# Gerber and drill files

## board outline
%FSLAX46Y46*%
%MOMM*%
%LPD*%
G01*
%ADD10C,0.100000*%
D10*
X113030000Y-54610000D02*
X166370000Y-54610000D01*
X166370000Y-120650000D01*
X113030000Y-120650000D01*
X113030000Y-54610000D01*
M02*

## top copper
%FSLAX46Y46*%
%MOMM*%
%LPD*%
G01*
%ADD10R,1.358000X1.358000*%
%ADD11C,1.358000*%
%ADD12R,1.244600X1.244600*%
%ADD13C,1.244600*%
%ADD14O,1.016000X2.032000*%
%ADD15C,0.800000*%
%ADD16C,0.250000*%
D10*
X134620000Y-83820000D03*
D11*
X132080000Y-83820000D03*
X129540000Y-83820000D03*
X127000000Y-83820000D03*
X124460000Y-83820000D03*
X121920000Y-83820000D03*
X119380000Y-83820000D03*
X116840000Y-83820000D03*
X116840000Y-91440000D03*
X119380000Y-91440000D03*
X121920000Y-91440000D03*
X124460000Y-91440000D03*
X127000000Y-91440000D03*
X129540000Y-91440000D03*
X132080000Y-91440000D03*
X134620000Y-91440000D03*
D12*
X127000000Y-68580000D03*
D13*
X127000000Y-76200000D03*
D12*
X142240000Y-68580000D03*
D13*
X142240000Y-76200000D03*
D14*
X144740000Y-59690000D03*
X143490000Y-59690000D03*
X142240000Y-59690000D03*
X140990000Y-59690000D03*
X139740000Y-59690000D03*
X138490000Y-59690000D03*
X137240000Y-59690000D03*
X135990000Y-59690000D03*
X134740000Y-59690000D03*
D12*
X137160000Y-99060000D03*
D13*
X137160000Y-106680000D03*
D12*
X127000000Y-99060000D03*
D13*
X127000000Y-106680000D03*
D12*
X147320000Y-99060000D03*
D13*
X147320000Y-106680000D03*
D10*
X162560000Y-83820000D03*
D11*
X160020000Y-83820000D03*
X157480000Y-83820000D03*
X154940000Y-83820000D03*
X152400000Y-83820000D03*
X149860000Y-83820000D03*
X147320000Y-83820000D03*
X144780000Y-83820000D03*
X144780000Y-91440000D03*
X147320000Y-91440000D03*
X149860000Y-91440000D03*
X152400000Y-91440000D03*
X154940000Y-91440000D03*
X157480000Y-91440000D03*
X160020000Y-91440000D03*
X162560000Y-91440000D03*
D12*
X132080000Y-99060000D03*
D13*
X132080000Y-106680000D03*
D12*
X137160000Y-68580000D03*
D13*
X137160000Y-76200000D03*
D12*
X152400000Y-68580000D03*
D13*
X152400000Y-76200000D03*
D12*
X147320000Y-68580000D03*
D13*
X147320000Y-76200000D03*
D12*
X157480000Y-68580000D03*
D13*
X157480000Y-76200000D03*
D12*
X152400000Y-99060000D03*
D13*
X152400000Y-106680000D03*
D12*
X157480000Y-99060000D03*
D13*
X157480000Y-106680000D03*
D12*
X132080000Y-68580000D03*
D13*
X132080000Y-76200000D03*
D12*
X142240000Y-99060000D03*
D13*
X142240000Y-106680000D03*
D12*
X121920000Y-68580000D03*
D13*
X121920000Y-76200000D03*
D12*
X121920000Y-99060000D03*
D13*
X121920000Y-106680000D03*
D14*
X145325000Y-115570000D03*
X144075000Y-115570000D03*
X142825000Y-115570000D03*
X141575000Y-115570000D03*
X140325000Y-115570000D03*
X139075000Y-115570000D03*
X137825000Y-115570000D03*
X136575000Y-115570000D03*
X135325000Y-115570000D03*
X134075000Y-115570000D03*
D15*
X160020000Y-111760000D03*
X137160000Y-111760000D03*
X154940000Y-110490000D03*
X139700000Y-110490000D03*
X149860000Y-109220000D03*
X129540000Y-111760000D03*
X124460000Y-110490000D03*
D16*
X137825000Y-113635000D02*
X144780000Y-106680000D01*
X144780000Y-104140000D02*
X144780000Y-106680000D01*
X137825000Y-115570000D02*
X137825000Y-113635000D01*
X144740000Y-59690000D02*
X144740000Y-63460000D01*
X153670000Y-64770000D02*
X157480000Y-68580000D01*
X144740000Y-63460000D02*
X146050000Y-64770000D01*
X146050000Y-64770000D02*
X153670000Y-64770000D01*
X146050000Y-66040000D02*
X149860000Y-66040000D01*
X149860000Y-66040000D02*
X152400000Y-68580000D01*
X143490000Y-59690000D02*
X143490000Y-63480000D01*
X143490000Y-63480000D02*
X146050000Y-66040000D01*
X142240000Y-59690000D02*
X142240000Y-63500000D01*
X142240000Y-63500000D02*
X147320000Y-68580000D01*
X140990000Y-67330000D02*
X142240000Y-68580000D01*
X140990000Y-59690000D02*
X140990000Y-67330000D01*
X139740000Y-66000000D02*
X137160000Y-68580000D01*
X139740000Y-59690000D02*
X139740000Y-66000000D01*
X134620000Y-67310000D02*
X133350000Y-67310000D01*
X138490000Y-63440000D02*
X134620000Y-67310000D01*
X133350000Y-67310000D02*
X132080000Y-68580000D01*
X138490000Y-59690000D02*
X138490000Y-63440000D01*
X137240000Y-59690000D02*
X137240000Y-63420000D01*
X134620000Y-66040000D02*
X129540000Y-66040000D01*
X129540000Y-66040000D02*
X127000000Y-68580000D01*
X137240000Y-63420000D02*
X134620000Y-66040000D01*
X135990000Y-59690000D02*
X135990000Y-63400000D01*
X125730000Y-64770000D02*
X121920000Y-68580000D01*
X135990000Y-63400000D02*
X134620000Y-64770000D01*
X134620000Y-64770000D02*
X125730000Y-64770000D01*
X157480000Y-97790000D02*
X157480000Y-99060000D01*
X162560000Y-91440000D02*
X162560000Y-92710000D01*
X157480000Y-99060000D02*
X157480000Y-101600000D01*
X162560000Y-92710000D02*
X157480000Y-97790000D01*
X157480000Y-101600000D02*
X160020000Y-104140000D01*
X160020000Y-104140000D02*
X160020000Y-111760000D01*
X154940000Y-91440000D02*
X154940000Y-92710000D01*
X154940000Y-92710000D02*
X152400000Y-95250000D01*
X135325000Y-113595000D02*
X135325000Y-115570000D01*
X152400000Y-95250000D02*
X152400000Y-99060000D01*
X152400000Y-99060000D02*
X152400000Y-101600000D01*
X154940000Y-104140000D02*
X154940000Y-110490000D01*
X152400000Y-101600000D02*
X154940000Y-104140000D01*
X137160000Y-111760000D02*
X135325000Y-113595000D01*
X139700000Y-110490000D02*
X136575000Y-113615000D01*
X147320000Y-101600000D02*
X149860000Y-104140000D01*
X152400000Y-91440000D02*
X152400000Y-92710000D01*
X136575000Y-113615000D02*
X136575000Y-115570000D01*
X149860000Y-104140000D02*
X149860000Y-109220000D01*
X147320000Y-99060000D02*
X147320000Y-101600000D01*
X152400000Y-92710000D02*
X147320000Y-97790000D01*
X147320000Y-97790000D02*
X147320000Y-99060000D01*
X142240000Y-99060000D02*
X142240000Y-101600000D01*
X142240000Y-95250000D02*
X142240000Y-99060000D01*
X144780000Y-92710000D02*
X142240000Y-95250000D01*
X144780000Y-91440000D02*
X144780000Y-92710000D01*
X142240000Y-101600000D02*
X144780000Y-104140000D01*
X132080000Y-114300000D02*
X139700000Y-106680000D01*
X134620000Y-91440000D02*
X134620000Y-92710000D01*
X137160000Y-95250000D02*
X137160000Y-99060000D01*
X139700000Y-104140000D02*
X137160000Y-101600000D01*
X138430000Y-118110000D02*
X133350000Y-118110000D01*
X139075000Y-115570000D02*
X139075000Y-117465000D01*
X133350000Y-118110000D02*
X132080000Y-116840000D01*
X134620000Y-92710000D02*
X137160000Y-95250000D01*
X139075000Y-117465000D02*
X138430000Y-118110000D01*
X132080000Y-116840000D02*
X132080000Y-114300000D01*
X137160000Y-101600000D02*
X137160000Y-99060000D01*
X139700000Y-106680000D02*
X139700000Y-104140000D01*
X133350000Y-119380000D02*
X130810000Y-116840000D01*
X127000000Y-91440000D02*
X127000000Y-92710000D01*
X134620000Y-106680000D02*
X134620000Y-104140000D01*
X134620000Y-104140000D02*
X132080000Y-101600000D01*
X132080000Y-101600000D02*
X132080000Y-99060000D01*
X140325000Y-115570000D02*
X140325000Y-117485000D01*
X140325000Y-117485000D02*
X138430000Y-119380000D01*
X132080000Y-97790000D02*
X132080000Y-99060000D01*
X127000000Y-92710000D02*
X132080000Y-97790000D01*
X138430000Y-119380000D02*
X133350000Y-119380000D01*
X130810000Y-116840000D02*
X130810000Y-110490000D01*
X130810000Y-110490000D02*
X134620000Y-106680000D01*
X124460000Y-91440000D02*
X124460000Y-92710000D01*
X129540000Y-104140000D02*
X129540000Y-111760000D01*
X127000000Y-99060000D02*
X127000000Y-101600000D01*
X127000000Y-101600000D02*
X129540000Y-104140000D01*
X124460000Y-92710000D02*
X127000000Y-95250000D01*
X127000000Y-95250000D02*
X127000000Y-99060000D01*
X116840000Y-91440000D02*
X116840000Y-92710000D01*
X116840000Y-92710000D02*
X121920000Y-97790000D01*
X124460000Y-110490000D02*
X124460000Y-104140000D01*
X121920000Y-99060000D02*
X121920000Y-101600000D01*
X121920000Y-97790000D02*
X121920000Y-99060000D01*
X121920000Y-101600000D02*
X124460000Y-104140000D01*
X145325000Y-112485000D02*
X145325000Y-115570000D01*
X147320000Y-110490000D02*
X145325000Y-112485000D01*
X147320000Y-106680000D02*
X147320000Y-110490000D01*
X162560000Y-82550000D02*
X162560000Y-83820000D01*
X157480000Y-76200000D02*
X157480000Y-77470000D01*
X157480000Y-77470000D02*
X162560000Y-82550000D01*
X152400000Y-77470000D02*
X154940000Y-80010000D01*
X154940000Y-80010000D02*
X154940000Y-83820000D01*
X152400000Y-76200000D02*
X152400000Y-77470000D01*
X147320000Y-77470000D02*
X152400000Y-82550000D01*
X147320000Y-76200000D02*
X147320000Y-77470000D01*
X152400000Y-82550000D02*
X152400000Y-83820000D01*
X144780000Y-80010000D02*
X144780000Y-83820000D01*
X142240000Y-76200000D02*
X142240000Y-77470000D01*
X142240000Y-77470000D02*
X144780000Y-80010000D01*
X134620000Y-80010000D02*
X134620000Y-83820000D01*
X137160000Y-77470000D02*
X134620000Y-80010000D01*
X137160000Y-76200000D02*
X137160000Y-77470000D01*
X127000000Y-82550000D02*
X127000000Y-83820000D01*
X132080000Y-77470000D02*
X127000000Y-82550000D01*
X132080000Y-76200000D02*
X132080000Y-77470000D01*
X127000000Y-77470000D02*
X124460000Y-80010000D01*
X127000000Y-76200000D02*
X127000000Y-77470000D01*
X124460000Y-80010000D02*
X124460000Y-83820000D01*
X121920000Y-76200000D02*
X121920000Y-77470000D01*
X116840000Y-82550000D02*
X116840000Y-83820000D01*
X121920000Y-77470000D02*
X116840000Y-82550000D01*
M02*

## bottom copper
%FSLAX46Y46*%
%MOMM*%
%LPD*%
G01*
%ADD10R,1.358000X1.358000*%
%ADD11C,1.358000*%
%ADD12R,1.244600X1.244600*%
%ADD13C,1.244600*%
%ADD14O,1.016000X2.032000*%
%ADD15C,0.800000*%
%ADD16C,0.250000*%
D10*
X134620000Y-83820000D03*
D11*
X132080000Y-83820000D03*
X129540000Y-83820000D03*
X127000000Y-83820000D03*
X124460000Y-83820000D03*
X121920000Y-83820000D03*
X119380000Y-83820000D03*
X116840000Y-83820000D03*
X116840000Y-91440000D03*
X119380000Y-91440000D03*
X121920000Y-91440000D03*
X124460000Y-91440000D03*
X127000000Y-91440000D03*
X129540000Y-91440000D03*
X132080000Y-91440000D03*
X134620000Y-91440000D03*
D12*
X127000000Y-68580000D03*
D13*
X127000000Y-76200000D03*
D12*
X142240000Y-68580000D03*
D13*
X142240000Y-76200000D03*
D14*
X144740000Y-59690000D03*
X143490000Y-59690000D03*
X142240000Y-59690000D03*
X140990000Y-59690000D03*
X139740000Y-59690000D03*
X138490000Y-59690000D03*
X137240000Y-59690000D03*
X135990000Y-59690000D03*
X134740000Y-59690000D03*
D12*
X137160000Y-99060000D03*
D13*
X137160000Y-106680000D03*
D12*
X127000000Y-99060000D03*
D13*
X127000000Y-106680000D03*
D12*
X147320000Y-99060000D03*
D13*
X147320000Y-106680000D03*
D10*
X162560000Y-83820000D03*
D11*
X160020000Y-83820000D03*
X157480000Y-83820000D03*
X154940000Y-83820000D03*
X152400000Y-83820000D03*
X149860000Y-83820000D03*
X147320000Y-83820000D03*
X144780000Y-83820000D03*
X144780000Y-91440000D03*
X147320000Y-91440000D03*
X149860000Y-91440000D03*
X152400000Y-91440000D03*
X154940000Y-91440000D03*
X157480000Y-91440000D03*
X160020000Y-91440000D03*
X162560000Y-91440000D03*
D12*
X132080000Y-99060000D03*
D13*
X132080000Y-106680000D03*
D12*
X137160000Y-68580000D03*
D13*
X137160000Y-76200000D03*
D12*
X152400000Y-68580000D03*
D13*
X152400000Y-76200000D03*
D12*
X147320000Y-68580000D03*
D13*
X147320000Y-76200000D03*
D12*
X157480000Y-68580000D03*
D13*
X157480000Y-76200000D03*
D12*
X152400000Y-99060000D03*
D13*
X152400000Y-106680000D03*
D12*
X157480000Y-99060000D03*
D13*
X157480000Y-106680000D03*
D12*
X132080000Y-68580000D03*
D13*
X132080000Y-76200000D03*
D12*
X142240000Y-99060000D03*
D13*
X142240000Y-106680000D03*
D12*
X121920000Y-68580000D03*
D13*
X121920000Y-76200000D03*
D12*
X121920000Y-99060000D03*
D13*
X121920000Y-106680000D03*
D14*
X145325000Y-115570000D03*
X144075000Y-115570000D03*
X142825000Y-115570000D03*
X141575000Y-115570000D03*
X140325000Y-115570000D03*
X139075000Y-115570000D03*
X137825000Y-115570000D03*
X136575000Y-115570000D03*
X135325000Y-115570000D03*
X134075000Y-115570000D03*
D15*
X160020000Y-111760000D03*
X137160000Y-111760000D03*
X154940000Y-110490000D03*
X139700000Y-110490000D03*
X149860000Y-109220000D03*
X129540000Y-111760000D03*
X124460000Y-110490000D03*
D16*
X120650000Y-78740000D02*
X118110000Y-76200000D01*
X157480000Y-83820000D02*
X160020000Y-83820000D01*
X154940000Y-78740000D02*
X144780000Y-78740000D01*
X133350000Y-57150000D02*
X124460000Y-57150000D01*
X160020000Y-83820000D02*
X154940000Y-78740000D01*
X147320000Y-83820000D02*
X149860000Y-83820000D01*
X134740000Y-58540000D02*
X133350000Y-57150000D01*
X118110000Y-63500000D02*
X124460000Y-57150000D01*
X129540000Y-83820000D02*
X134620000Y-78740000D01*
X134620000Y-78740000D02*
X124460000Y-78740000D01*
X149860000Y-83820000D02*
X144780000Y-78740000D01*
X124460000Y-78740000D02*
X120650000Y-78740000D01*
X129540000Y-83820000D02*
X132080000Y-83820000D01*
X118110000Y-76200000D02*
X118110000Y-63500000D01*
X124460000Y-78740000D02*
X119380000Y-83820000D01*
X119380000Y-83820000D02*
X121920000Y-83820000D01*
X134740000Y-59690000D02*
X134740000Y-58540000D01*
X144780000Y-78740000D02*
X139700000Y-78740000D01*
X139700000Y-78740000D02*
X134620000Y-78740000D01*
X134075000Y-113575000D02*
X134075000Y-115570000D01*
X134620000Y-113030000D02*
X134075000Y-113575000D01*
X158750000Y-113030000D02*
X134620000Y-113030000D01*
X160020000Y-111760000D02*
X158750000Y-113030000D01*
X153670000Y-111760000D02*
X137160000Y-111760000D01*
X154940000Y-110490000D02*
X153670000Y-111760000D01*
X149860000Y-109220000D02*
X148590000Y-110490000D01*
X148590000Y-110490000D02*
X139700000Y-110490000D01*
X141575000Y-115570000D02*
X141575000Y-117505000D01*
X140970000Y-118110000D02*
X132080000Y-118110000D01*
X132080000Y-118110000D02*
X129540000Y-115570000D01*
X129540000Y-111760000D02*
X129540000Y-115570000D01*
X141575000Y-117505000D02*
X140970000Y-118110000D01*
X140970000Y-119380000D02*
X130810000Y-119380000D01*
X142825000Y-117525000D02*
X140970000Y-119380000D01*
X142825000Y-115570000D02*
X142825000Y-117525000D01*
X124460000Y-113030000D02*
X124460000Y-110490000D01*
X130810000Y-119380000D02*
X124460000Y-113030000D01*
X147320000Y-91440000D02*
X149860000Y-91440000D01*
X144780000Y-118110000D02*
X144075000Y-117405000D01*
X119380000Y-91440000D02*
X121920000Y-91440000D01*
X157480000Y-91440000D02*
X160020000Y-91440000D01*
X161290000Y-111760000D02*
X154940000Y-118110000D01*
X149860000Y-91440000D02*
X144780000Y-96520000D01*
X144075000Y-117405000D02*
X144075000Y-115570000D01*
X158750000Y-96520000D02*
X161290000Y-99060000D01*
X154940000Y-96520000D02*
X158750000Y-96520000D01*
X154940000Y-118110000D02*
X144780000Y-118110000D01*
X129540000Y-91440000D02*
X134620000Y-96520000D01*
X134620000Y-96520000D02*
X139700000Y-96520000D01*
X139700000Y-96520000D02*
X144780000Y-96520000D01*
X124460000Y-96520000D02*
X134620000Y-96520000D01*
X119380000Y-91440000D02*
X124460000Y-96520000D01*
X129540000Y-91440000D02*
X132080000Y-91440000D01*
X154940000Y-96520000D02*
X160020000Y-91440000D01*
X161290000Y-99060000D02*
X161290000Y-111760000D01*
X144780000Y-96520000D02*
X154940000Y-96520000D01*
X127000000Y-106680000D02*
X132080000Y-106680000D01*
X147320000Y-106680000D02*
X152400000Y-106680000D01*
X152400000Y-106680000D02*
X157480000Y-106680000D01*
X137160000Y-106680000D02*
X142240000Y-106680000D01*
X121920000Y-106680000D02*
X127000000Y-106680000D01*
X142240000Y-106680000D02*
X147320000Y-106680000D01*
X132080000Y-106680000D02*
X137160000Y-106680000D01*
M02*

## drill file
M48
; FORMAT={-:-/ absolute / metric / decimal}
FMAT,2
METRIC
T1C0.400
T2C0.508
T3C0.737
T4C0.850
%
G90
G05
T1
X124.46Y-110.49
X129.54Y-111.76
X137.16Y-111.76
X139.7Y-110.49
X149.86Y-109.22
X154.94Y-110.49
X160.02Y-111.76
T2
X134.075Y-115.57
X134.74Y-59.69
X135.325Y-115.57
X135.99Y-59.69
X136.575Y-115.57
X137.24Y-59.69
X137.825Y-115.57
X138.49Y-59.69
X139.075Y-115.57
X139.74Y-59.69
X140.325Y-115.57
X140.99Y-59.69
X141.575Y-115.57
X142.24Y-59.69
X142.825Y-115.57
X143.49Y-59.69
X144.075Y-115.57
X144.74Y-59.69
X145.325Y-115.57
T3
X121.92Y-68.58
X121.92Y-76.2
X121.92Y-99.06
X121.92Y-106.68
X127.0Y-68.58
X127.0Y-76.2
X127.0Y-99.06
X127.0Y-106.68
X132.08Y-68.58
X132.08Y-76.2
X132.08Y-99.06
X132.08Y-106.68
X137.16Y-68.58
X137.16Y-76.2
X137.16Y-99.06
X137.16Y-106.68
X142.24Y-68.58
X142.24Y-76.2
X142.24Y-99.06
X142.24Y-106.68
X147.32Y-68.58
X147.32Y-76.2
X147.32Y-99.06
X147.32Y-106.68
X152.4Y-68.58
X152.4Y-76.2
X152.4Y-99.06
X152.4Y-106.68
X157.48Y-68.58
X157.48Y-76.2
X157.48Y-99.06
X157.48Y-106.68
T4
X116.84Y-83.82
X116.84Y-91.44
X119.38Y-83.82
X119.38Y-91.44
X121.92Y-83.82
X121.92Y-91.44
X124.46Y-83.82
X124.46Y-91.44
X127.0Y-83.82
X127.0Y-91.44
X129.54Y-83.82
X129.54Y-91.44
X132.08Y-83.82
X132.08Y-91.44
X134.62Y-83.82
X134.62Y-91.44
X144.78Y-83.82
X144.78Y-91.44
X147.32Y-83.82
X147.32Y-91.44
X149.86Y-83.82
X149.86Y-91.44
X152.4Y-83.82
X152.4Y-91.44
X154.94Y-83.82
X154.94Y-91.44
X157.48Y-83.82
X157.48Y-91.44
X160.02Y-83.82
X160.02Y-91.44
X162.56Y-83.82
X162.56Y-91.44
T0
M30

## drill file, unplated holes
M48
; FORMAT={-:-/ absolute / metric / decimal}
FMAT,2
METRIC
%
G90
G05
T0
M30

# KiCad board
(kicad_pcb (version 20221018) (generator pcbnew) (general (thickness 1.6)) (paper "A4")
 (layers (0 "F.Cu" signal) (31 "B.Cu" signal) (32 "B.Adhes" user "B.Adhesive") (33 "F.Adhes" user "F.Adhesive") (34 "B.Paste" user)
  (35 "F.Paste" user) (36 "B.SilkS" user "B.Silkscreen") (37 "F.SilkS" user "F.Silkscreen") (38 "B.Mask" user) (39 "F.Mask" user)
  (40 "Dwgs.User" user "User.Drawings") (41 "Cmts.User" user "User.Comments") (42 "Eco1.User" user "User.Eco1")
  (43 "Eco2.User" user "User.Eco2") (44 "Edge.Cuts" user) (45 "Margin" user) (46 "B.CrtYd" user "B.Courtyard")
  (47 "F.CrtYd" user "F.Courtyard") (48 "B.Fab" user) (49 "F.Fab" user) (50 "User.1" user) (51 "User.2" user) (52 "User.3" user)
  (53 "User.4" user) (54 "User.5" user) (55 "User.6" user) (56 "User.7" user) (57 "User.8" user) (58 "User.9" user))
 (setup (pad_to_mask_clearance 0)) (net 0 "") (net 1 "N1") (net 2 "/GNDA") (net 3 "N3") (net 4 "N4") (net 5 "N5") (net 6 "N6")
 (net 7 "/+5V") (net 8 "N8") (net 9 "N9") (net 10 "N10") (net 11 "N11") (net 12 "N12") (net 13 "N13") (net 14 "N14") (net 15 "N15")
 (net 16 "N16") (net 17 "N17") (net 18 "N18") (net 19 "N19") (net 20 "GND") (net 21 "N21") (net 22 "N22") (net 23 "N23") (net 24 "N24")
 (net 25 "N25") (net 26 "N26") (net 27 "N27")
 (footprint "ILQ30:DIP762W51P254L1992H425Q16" (layer "F.Cu") (at 125.73 87.63 -90)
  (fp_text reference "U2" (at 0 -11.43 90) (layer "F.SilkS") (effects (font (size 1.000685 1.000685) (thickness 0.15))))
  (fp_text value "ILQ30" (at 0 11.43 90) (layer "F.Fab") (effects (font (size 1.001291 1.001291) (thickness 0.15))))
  (pad "1" thru_hole rect (at -3.81 -8.89 270) (size 1.358 1.358) (drill 0.85) (layers "*.Cu" "*.Mask") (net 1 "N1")
   (solder_mask_margin 0.102))
  (pad "2" thru_hole circle (at -3.81 -6.35 270) (size 1.358 1.358) (drill 0.85) (layers "*.Cu" "*.Mask") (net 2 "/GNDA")
   (solder_mask_margin 0.102))
  (pad "3" thru_hole circle (at -3.81 -3.81 270) (size 1.358 1.358) (drill 0.85) (layers "*.Cu" "*.Mask") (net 2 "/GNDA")
   (solder_mask_margin 0.102))
  (pad "4" thru_hole circle (at -3.81 -1.27 270) (size 1.358 1.358) (drill 0.85) (layers "*.Cu" "*.Mask") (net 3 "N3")
   (solder_mask_margin 0.102))
  (pad "5" thru_hole circle (at -3.81 1.27 270) (size 1.358 1.358) (drill 0.85) (layers "*.Cu" "*.Mask") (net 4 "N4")
   (solder_mask_margin 0.102))
  (pad "6" thru_hole circle (at -3.81 3.81 270) (size 1.358 1.358) (drill 0.85) (layers "*.Cu" "*.Mask") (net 2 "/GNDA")
   (solder_mask_margin 0.102))
  (pad "7" thru_hole circle (at -3.81 6.35 270) (size 1.358 1.358) (drill 0.85) (layers "*.Cu" "*.Mask") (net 2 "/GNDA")
   (solder_mask_margin 0.102))
  (pad "8" thru_hole circle (at -3.81 8.89 270) (size 1.358 1.358) (drill 0.85) (layers "*.Cu" "*.Mask") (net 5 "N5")
   (solder_mask_margin 0.102))
  (pad "9" thru_hole circle (at 3.81 8.89 270) (size 1.358 1.358) (drill 0.85) (layers "*.Cu" "*.Mask") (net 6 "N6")
   (solder_mask_margin 0.102))
  (pad "10" thru_hole circle (at 3.81 6.35 270) (size 1.358 1.358) (drill 0.85) (layers "*.Cu" "*.Mask") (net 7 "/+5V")
   (solder_mask_margin 0.102))
  (pad "11" thru_hole circle (at 3.81 3.81 270) (size 1.358 1.358) (drill 0.85) (layers "*.Cu" "*.Mask") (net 7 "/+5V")
   (solder_mask_margin 0.102))
  (pad "12" thru_hole circle (at 3.81 1.27 270) (size 1.358 1.358) (drill 0.85) (layers "*.Cu" "*.Mask") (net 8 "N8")
   (solder_mask_margin 0.102))
  (pad "13" thru_hole circle (at 3.81 -1.27 270) (size 1.358 1.358) (drill 0.85) (layers "*.Cu" "*.Mask") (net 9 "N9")
   (solder_mask_margin 0.102))
  (pad "14" thru_hole circle (at 3.81 -3.81 270) (size 1.358 1.358) (drill 0.85) (layers "*.Cu" "*.Mask") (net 7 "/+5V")
   (solder_mask_margin 0.102))
  (pad "15" thru_hole circle (at 3.81 -6.35 270) (size 1.358 1.358) (drill 0.85) (layers "*.Cu" "*.Mask") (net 7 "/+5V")
   (solder_mask_margin 0.102))
  (pad "16" thru_hole circle (at 3.81 -8.89 270) (size 1.358 1.358) (drill 0.85) (layers "*.Cu" "*.Mask") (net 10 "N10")
   (solder_mask_margin 0.102)))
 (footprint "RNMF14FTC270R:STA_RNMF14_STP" (layer "F.Cu") (at 127 68.58 -90)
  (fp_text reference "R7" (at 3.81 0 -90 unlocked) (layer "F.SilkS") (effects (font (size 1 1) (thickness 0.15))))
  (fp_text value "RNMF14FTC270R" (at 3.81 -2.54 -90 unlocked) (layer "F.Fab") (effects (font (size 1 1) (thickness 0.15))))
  (pad "1" thru_hole rect (at 0 0 270) (size 1.2446 1.2446) (drill 0.7366) (layers "*.Cu" "*.Mask") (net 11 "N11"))
  (pad "2" thru_hole circle (at 7.62 0 270) (size 1.2446 1.2446) (drill 0.7366) (layers "*.Cu" "*.Mask") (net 4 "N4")))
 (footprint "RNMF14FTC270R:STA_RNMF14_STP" (layer "F.Cu") (at 142.24 68.58 -90)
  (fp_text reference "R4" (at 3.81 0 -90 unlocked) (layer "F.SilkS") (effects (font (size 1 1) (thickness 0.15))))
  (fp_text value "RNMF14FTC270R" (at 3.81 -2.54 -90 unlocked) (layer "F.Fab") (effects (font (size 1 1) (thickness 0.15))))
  (pad "1" thru_hole rect (at 0 0 270) (size 1.2446 1.2446) (drill 0.7366) (layers "*.Cu" "*.Mask") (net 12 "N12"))
  (pad "2" thru_hole circle (at 7.62 0 270) (size 1.2446 1.2446) (drill 0.7366) (layers "*.Cu" "*.Mask") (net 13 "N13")))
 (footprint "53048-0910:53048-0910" (layer "F.Cu") (at 139.74 59.69 180)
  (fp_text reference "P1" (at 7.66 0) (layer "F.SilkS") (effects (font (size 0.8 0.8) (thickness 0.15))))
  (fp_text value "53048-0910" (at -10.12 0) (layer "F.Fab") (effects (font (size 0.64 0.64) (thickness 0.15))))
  (pad "1" thru_hole oval (at -5 0 180) (size 1.016 2.032) (drill 0.508) (layers "*.Cu" "*.Mask") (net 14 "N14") (solder_mask_margin 0.102))
  (pad "2" thru_hole oval (at -3.75 0 180) (size 1.016 2.032) (drill 0.508) (layers "*.Cu" "*.Mask") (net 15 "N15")
   (solder_mask_margin 0.102))
  (pad "3" thru_hole oval (at -2.5 0 180) (size 1.016 2.032) (drill 0.508) (layers "*.Cu" "*.Mask") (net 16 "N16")
   (solder_mask_margin 0.102))
  (pad "4" thru_hole oval (at -1.25 0 180) (size 1.016 2.032) (drill 0.508) (layers "*.Cu" "*.Mask") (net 12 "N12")
   (solder_mask_margin 0.102))
  (pad "5" thru_hole oval (at 0 0 180) (size 1.016 2.032) (drill 0.508) (layers "*.Cu" "*.Mask") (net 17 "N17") (solder_mask_margin 0.102))
  (pad "6" thru_hole oval (at 1.25 0 180) (size 1.016 2.032) (drill 0.508) (layers "*.Cu" "*.Mask") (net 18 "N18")
   (solder_mask_margin 0.102))
  (pad "7" thru_hole oval (at 2.5 0 180) (size 1.016 2.032) (drill 0.508) (layers "*.Cu" "*.Mask") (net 11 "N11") (solder_mask_margin 0.102))
  (pad "8" thru_hole oval (at 3.75 0 180) (size 1.016 2.032) (drill 0.508) (layers "*.Cu" "*.Mask") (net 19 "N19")
   (solder_mask_margin 0.102))
  (pad "9" thru_hole oval (at 5 0 180) (size 1.016 2.032) (drill 0.508) (layers "*.Cu" "*.Mask") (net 2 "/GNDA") (solder_mask_margin 0.102)))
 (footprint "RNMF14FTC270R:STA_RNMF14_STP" (layer "F.Cu") (at 137.16 99.06 -90)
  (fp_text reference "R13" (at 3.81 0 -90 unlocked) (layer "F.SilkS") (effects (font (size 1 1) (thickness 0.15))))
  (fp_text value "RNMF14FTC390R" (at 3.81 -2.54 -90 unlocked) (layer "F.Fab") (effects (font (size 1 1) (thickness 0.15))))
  (pad "1" thru_hole rect (at 0 0 270) (size 1.2446 1.2446) (drill 0.7366) (layers "*.Cu" "*.Mask") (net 10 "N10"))
  (pad "2" thru_hole circle (at 7.62 0 270) (size 1.2446 1.2446) (drill 0.7366) (layers "*.Cu" "*.Mask") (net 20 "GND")))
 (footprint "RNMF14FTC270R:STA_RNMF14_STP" (layer "F.Cu") (at 127 99.06 -90)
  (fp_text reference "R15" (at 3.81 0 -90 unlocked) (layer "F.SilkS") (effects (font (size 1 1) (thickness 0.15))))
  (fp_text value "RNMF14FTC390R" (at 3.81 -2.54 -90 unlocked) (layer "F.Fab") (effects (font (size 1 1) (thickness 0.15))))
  (pad "1" thru_hole rect (at 0 0 270) (size 1.2446 1.2446) (drill 0.7366) (layers "*.Cu" "*.Mask") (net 8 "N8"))
  (pad "2" thru_hole circle (at 7.62 0 270) (size 1.2446 1.2446) (drill 0.7366) (layers "*.Cu" "*.Mask") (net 20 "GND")))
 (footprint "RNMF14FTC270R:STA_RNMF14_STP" (layer "F.Cu") (at 147.32 99.06 -90)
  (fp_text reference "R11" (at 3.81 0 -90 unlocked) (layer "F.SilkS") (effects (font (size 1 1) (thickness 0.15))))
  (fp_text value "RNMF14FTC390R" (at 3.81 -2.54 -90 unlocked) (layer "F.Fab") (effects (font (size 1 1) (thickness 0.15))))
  (pad "1" thru_hole rect (at 0 0 270) (size 1.2446 1.2446) (drill 0.7366) (layers "*.Cu" "*.Mask") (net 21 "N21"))
  (pad "2" thru_hole circle (at 7.62 0 270) (size 1.2446 1.2446) (drill 0.7366) (layers "*.Cu" "*.Mask") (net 20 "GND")))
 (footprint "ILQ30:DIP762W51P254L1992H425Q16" (layer "F.Cu") (at 153.67 87.63 -90)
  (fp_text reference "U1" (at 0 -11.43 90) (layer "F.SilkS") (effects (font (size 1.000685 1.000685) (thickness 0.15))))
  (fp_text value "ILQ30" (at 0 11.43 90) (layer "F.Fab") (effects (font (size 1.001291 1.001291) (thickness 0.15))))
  (pad "1" thru_hole rect (at -3.81 -8.89 270) (size 1.358 1.358) (drill 0.85) (layers "*.Cu" "*.Mask") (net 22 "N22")
   (solder_mask_margin 0.102))
  (pad "2" thru_hole circle (at -3.81 -6.35 270) (size 1.358 1.358) (drill 0.85) (layers "*.Cu" "*.Mask") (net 2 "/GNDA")
   (solder_mask_margin 0.102))
  (pad "3" thru_hole circle (at -3.81 -3.81 270) (size 1.358 1.358) (drill 0.85) (layers "*.Cu" "*.Mask") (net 2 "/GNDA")
   (solder_mask_margin 0.102))
  (pad "4" thru_hole circle (at -3.81 -1.27 270) (size 1.358 1.358) (drill 0.85) (layers "*.Cu" "*.Mask") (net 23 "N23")
   (solder_mask_margin 0.102))
  (pad "5" thru_hole circle (at -3.81 1.27 270) (size 1.358 1.358) (drill 0.85) (layers "*.Cu" "*.Mask") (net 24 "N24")
   (solder_mask_margin 0.102))
  (pad "6" thru_hole circle (at -3.81 3.81 270) (size 1.358 1.358) (drill 0.85) (layers "*.Cu" "*.Mask") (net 2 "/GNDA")
   (solder_mask_margin 0.102))
  (pad "7" thru_hole circle (at -3.81 6.35 270) (size 1.358 1.358) (drill 0.85) (layers "*.Cu" "*.Mask") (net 2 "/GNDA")
   (solder_mask_margin 0.102))
  (pad "8" thru_hole circle (at -3.81 8.89 270) (size 1.358 1.358) (drill 0.85) (layers "*.Cu" "*.Mask") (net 13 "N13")
   (solder_mask_margin 0.102))
  (pad "9" thru_hole circle (at 3.81 8.89 270) (size 1.358 1.358) (drill 0.85) (layers "*.Cu" "*.Mask") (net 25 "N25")
   (solder_mask_margin 0.102))
  (pad "10" thru_hole circle (at 3.81 6.35 270) (size 1.358 1.358) (drill 0.85) (layers "*.Cu" "*.Mask") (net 7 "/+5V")
   (solder_mask_margin 0.102))
  (pad "11" thru_hole circle (at 3.81 3.81 270) (size 1.358 1.358) (drill 0.85) (layers "*.Cu" "*.Mask") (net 7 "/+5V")
   (solder_mask_margin 0.102))
  (pad "12" thru_hole circle (at 3.81 1.27 270) (size 1.358 1.358) (drill 0.85) (layers "*.Cu" "*.Mask") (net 21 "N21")
   (solder_mask_margin 0.102))
  (pad "13" thru_hole circle (at 3.81 -1.27 270) (size 1.358 1.358) (drill 0.85) (layers "*.Cu" "*.Mask") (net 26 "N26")
   (solder_mask_margin 0.102))
  (pad "14" thru_hole circle (at 3.81 -3.81 270) (size 1.358 1.358) (drill 0.85) (layers "*.Cu" "*.Mask") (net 7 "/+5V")
   (solder_mask_margin 0.102))
  (pad "15" thru_hole circle (at 3.81 -6.35 270) (size 1.358 1.358) (drill 0.85) (layers "*.Cu" "*.Mask") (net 7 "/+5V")
   (solder_mask_margin 0.102))
  (pad "16" thru_hole circle (at 3.81 -8.89 270) (size 1.358 1.358) (drill 0.85) (layers "*.Cu" "*.Mask") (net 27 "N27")
   (solder_mask_margin 0.102)))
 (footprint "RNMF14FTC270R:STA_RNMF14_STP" (layer "F.Cu") (at 132.08 99.06 -90)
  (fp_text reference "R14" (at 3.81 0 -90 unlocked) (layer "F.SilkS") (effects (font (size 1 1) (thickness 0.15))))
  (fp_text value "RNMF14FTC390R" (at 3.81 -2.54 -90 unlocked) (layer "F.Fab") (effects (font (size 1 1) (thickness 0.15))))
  (pad "1" thru_hole rect (at 0 0 270) (size 1.2446 1.2446) (drill 0.7366) (layers "*.Cu" "*.Mask") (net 9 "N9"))
  (pad "2" thru_hole circle (at 7.62 0 270) (size 1.2446 1.2446) (drill 0.7366) (layers "*.Cu" "*.Mask") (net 20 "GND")))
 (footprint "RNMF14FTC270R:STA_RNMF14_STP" (layer "F.Cu") (at 137.16 68.58 -90)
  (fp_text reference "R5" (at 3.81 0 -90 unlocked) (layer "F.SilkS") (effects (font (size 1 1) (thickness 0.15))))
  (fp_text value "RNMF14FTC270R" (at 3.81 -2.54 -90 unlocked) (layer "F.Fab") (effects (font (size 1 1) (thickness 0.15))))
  (pad "1" thru_hole rect (at 0 0 270) (size 1.2446 1.2446) (drill 0.7366) (layers "*.Cu" "*.Mask") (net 17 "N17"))
  (pad "2" thru_hole circle (at 7.62 0 270) (size 1.2446 1.2446) (drill 0.7366) (layers "*.Cu" "*.Mask") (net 1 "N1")))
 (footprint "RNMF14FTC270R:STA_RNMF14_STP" (layer "F.Cu") (at 152.4 68.58 -90)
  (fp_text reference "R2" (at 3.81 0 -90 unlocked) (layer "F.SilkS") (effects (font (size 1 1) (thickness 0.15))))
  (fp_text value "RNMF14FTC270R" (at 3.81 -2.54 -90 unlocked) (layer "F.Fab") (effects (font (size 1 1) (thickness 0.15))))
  (pad "1" thru_hole rect (at 0 0 270) (size 1.2446 1.2446) (drill 0.7366) (layers "*.Cu" "*.Mask") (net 15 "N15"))
  (pad "2" thru_hole circle (at 7.62 0 270) (size 1.2446 1.2446) (drill 0.7366) (layers "*.Cu" "*.Mask") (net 23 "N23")))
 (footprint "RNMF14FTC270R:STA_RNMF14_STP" (layer "F.Cu") (at 147.32 68.58 -90)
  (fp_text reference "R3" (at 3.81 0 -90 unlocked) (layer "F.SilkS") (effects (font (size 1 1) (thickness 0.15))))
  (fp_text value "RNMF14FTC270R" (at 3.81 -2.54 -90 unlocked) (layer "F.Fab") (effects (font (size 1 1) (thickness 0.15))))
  (pad "1" thru_hole rect (at 0 0 270) (size 1.2446 1.2446) (drill 0.7366) (layers "*.Cu" "*.Mask") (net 16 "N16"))
  (pad "2" thru_hole circle (at 7.62 0 270) (size 1.2446 1.2446) (drill 0.7366) (layers "*.Cu" "*.Mask") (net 24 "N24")))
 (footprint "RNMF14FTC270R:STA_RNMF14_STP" (layer "F.Cu") (at 157.48 68.58 -90)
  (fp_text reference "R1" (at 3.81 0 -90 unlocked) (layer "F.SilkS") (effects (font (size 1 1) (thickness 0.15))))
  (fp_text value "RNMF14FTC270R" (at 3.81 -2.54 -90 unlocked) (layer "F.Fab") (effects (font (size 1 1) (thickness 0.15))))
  (pad "1" thru_hole rect (at 0 0 270) (size 1.2446 1.2446) (drill 0.7366) (layers "*.Cu" "*.Mask") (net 14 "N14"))
  (pad "2" thru_hole circle (at 7.62 0 270) (size 1.2446 1.2446) (drill 0.7366) (layers "*.Cu" "*.Mask") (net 22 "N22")))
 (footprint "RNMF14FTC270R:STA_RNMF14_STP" (layer "F.Cu") (at 152.4 99.06 -90)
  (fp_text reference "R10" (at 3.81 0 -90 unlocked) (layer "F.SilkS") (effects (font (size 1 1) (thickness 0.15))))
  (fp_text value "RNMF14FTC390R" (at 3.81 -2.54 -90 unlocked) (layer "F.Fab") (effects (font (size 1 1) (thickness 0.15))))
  (pad "1" thru_hole rect (at 0 0 270) (size 1.2446 1.2446) (drill 0.7366) (layers "*.Cu" "*.Mask") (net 26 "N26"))
  (pad "2" thru_hole circle (at 7.62 0 270) (size 1.2446 1.2446) (drill 0.7366) (layers "*.Cu" "*.Mask") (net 20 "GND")))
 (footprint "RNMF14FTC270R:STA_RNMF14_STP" (layer "F.Cu") (at 157.48 99.06 -90)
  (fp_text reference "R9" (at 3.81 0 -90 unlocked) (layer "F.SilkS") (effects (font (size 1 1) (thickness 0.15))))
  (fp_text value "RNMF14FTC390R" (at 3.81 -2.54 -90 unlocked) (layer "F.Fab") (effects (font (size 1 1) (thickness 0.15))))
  (pad "1" thru_hole rect (at 0 0 270) (size 1.2446 1.2446) (drill 0.7366) (layers "*.Cu" "*.Mask") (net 27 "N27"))
  (pad "2" thru_hole circle (at 7.62 0 270) (size 1.2446 1.2446) (drill 0.7366) (layers "*.Cu" "*.Mask") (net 20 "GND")))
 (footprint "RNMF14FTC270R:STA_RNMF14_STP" (layer "F.Cu") (at 132.08 68.58 -90)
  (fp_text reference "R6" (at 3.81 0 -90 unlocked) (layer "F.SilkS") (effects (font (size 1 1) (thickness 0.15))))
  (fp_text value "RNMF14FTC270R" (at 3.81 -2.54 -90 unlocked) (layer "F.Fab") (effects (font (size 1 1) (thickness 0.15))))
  (pad "1" thru_hole rect (at 0 0 270) (size 1.2446 1.2446) (drill 0.7366) (layers "*.Cu" "*.Mask") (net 18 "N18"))
  (pad "2" thru_hole circle (at 7.62 0 270) (size 1.2446 1.2446) (drill 0.7366) (layers "*.Cu" "*.Mask") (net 3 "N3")))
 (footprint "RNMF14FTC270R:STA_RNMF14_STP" (layer "F.Cu") (at 142.24 99.06 -90)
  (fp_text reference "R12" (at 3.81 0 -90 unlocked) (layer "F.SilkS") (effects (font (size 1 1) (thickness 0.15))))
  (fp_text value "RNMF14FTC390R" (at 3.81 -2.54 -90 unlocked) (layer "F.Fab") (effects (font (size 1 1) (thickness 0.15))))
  (pad "1" thru_hole rect (at 0 0 270) (size 1.2446 1.2446) (drill 0.7366) (layers "*.Cu" "*.Mask") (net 25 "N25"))
  (pad "2" thru_hole circle (at 7.62 0 270) (size 1.2446 1.2446) (drill 0.7366) (layers "*.Cu" "*.Mask") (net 20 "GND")))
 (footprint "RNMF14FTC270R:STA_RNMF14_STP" (layer "F.Cu") (at 121.92 68.58 -90)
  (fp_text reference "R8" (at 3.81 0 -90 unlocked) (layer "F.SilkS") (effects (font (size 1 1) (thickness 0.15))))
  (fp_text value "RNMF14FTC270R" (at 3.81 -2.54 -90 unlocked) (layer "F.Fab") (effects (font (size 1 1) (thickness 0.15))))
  (pad "1" thru_hole rect (at 0 0 270) (size 1.2446 1.2446) (drill 0.7366) (layers "*.Cu" "*.Mask") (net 19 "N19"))
  (pad "2" thru_hole circle (at 7.62 0 270) (size 1.2446 1.2446) (drill 0.7366) (layers "*.Cu" "*.Mask") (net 5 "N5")))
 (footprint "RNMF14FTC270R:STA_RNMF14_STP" (layer "F.Cu") (at 121.92 99.06 -90)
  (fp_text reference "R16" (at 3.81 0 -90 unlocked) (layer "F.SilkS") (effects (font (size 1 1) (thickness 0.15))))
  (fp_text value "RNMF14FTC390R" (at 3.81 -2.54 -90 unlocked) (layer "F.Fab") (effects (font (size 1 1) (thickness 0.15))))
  (pad "1" thru_hole rect (at 0 0 270) (size 1.2446 1.2446) (drill 0.7366) (layers "*.Cu" "*.Mask") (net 6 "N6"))
  (pad "2" thru_hole circle (at 7.62 0 270) (size 1.2446 1.2446) (drill 0.7366) (layers "*.Cu" "*.Mask") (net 20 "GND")))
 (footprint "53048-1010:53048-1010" (layer "F.Cu") (at 139.7 115.57)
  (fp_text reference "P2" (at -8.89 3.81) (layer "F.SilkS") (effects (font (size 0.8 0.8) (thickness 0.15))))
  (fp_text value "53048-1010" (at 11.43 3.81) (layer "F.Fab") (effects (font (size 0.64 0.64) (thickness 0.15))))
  (pad "1" thru_hole oval (at -5.625 0) (size 1.016 2.032) (drill 0.508) (layers "*.Cu" "*.Mask") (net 27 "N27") (solder_mask_margin 0.102))
  (pad "2" thru_hole oval (at -4.375 0) (size 1.016 2.032) (drill 0.508) (layers "*.Cu" "*.Mask") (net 26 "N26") (solder_mask_margin 0.102))
  (pad "3" thru_hole oval (at -3.125 0) (size 1.016 2.032) (drill 0.508) (layers "*.Cu" "*.Mask") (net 21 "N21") (solder_mask_margin 0.102))
  (pad "4" thru_hole oval (at -1.875 0) (size 1.016 2.032) (drill 0.508) (layers "*.Cu" "*.Mask") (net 25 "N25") (solder_mask_margin 0.102))
  (pad "5" thru_hole oval (at -0.625 0) (size 1.016 2.032) (drill 0.508) (layers "*.Cu" "*.Mask") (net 10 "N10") (solder_mask_margin 0.102))
  (pad "6" thru_hole oval (at 0.625 0) (size 1.016 2.032) (drill 0.508) (layers "*.Cu" "*.Mask") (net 9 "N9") (solder_mask_margin 0.102))
  (pad "7" thru_hole oval (at 1.875 0) (size 1.016 2.032) (drill 0.508) (layers "*.Cu" "*.Mask") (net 8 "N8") (solder_mask_margin 0.102))
  (pad "8" thru_hole oval (at 3.125 0) (size 1.016 2.032) (drill 0.508) (layers "*.Cu" "*.Mask") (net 6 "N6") (solder_mask_margin 0.102))
  (pad "9" thru_hole oval (at 4.375 0) (size 1.016 2.032) (drill 0.508) (layers "*.Cu" "*.Mask") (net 7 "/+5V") (solder_mask_margin 0.102))
  (pad "10" thru_hole oval (at 5.625 0) (size 1.016 2.032) (drill 0.508) (layers "*.Cu" "*.Mask") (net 20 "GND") (solder_mask_margin 0.102)))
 (gr_rect (start 113.03 54.61) (end 166.37 120.65) (stroke (width 0.1) (type default)) (fill none) (layer "Edge.Cuts"))
 (segment (start 144.74 59.69) (end 144.74 63.46) (width 0.25) (layer "F.Cu") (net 14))
 (segment (start 153.67 64.77) (end 157.48 68.58) (width 0.25) (layer "F.Cu") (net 14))
 (segment (start 144.74 63.46) (end 146.05 64.77) (width 0.25) (layer "F.Cu") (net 14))
 (segment (start 146.05 64.77) (end 153.67 64.77) (width 0.25) (layer "F.Cu") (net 14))
 (segment (start 146.05 66.04) (end 149.86 66.04) (width 0.25) (layer "F.Cu") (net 15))
 (segment (start 149.86 66.04) (end 152.4 68.58) (width 0.25) (layer "F.Cu") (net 15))
 (segment (start 143.49 59.69) (end 143.49 63.48) (width 0.25) (layer "F.Cu") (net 15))
 (segment (start 143.49 63.48) (end 146.05 66.04) (width 0.25) (layer "F.Cu") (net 15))
 (segment (start 142.24 59.69) (end 142.24 63.5) (width 0.25) (layer "F.Cu") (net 16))
 (segment (start 142.24 63.5) (end 147.32 68.58) (width 0.25) (layer "F.Cu") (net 16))
 (segment (start 140.99 67.33) (end 142.24 68.58) (width 0.25) (layer "F.Cu") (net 12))
 (segment (start 140.99 59.69) (end 140.99 67.33) (width 0.25) (layer "F.Cu") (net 12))
 (segment (start 139.74 66) (end 137.16 68.58) (width 0.25) (layer "F.Cu") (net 17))
 (segment (start 139.74 59.69) (end 139.74 66) (width 0.25) (layer "F.Cu") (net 17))
 (segment (start 134.62 67.31) (end 133.35 67.31) (width 0.25) (layer "F.Cu") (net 18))
 (segment (start 138.49 63.44) (end 134.62 67.31) (width 0.25) (layer "F.Cu") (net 18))
 (segment (start 133.35 67.31) (end 132.08 68.58) (width 0.25) (layer "F.Cu") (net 18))
 (segment (start 138.49 59.69) (end 138.49 63.44) (width 0.25) (layer "F.Cu") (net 18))
 (segment (start 137.24 59.69) (end 137.24 63.42) (width 0.25) (layer "F.Cu") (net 11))
 (segment (start 134.62 66.04) (end 129.54 66.04) (width 0.25) (layer "F.Cu") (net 11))
 (segment (start 129.54 66.04) (end 127 68.58) (width 0.25) (layer "F.Cu") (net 11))
 (segment (start 137.24 63.42) (end 134.62 66.04) (width 0.25) (layer "F.Cu") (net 11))
 (segment (start 135.99 59.69) (end 135.99 63.4) (width 0.25) (layer "F.Cu") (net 19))
 (segment (start 125.73 64.77) (end 121.92 68.58) (width 0.25) (layer "F.Cu") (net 19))
 (segment (start 135.99 63.4) (end 134.62 64.77) (width 0.25) (layer "F.Cu") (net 19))
 (segment (start 134.62 64.77) (end 125.73 64.77) (width 0.25) (layer "F.Cu") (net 19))
 (segment (start 120.65 78.74) (end 118.11 76.2) (width 0.25) (layer "B.Cu") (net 2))
 (segment (start 157.48 83.82) (end 160.02 83.82) (width 0.25) (layer "B.Cu") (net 2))
 (segment (start 154.94 78.74) (end 144.78 78.74) (width 0.25) (layer "B.Cu") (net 2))
 (segment (start 133.35 57.15) (end 124.46 57.15) (width 0.25) (layer "B.Cu") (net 2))
 (segment (start 160.02 83.82) (end 154.94 78.74) (width 0.25) (layer "B.Cu") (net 2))
 (segment (start 147.32 83.82) (end 149.86 83.82) (width 0.25) (layer "B.Cu") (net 2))
 (segment (start 134.74 58.54) (end 133.35 57.15) (width 0.25) (layer "B.Cu") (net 2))
 (segment (start 118.11 63.5) (end 124.46 57.15) (width 0.25) (layer "B.Cu") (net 2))
 (segment (start 129.54 83.82) (end 134.62 78.74) (width 0.25) (layer "B.Cu") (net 2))
 (segment (start 134.62 78.74) (end 124.46 78.74) (width 0.25) (layer "B.Cu") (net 2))
 (segment (start 149.86 83.82) (end 144.78 78.74) (width 0.25) (layer "B.Cu") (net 2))
 (segment (start 124.46 78.74) (end 120.65 78.74) (width 0.25) (layer "B.Cu") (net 2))
 (segment (start 129.54 83.82) (end 132.08 83.82) (width 0.25) (layer "B.Cu") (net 2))
 (segment (start 118.11 76.2) (end 118.11 63.5) (width 0.25) (layer "B.Cu") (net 2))
 (segment (start 124.46 78.74) (end 119.38 83.82) (width 0.25) (layer "B.Cu") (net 2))
 (segment (start 119.38 83.82) (end 121.92 83.82) (width 0.25) (layer "B.Cu") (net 2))
 (segment (start 134.74 59.69) (end 134.74 58.54) (width 0.25) (layer "B.Cu") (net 2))
 (segment (start 144.78 78.74) (end 139.7 78.74) (width 0.25) (layer "B.Cu") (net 2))
 (segment (start 139.7 78.74) (end 134.62 78.74) (width 0.25) (layer "B.Cu") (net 2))
 (segment (start 157.48 97.79) (end 157.48 99.06) (width 0.25) (layer "F.Cu") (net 27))
 (segment (start 162.56 91.44) (end 162.56 92.71) (width 0.25) (layer "F.Cu") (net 27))
 (segment (start 157.48 99.06) (end 157.48 101.6) (width 0.25) (layer "F.Cu") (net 27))
 (segment (start 162.56 92.71) (end 157.48 97.79) (width 0.25) (layer "F.Cu") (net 27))
 (segment (start 157.48 101.6) (end 160.02 104.14) (width 0.25) (layer "F.Cu") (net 27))
 (segment (start 160.02 104.14) (end 160.02 111.76) (width 0.25) (layer "F.Cu") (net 27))
 (via (at 160.02 111.76) (size 0.8) (drill 0.4) (layers "F.Cu" "B.Cu") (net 27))
 (segment (start 134.075 113.575) (end 134.075 115.57) (width 0.25) (layer "B.Cu") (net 27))
 (segment (start 134.62 113.03) (end 134.075 113.575) (width 0.25) (layer "B.Cu") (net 27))
 (segment (start 158.75 113.03) (end 134.62 113.03) (width 0.25) (layer "B.Cu") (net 27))
 (segment (start 160.02 111.76) (end 158.75 113.03) (width 0.25) (layer "B.Cu") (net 27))
 (segment (start 154.94 91.44) (end 154.94 92.71) (width 0.25) (layer "F.Cu") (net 26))
 (segment (start 154.94 92.71) (end 152.4 95.25) (width 0.25) (layer "F.Cu") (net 26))
 (segment (start 135.325 113.595) (end 135.325 115.57) (width 0.25) (layer "F.Cu") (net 26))
 (segment (start 152.4 95.25) (end 152.4 99.06) (width 0.25) (layer "F.Cu") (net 26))
 (segment (start 152.4 99.06) (end 152.4 101.6) (width 0.25) (layer "F.Cu") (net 26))
 (segment (start 154.94 104.14) (end 154.94 110.49) (width 0.25) (layer "F.Cu") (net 26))
 (segment (start 152.4 101.6) (end 154.94 104.14) (width 0.25) (layer "F.Cu") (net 26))
 (segment (start 137.16 111.76) (end 135.325 113.595) (width 0.25) (layer "F.Cu") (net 26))
 (via (at 137.16 111.76) (size 0.8) (drill 0.4) (layers "F.Cu" "B.Cu") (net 26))
 (via (at 154.94 110.49) (size 0.8) (drill 0.4) (layers "F.Cu" "B.Cu") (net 26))
 (segment (start 153.67 111.76) (end 137.16 111.76) (width 0.25) (layer "B.Cu") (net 26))
 (segment (start 154.94 110.49) (end 153.67 111.76) (width 0.25) (layer "B.Cu") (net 26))
 (segment (start 139.7 110.49) (end 136.575 113.615) (width 0.25) (layer "F.Cu") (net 21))
 (segment (start 147.32 101.6) (end 149.86 104.14) (width 0.25) (layer "F.Cu") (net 21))
 (segment (start 152.4 91.44) (end 152.4 92.71) (width 0.25) (layer "F.Cu") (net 21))
 (segment (start 136.575 113.615) (end 136.575 115.57) (width 0.25) (layer "F.Cu") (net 21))
 (segment (start 149.86 104.14) (end 149.86 109.22) (width 0.25) (layer "F.Cu") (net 21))
 (segment (start 147.32 99.06) (end 147.32 101.6) (width 0.25) (layer "F.Cu") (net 21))
 (segment (start 152.4 92.71) (end 147.32 97.79) (width 0.25) (layer "F.Cu") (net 21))
 (segment (start 147.32 97.79) (end 147.32 99.06) (width 0.25) (layer "F.Cu") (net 21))
 (via (at 139.7 110.49) (size 0.8) (drill 0.4) (layers "F.Cu" "B.Cu") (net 21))
 (via (at 149.86 109.22) (size 0.8) (drill 0.4) (layers "F.Cu" "B.Cu") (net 21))
 (segment (start 149.86 109.22) (end 148.59 110.49) (width 0.25) (layer "B.Cu") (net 21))
 (segment (start 148.59 110.49) (end 139.7 110.49) (width 0.25) (layer "B.Cu") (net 21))
 (segment (start 142.24 99.06) (end 142.24 101.6) (width 0.25) (layer "F.Cu") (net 25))
 (segment (start 142.24 95.25) (end 142.24 99.06) (width 0.25) (layer "F.Cu") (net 25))
 (segment (start 144.78 104.14) (end 144.78 106.68) (width 0.25) (layer "F.Cu") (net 25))
 (segment (start 144.78 92.71) (end 142.24 95.25) (width 0.25) (layer "F.Cu") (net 25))
 (segment (start 144.78 91.44) (end 144.78 92.71) (width 0.25) (layer "F.Cu") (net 25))
 (segment (start 137.825 113.635) (end 144.78 106.68) (width 0.25) (layer "F.Cu") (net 25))
 (segment (start 137.825 115.57) (end 137.825 113.635) (width 0.25) (layer "F.Cu") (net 25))
 (segment (start 142.24 101.6) (end 144.78 104.14) (width 0.25) (layer "F.Cu") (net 25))
 (segment (start 132.08 114.3) (end 139.7 106.68) (width 0.25) (layer "F.Cu") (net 10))
 (segment (start 134.62 91.44) (end 134.62 92.71) (width 0.25) (layer "F.Cu") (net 10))
 (segment (start 137.16 95.25) (end 137.16 99.06) (width 0.25) (layer "F.Cu") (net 10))
 (segment (start 139.7 104.14) (end 137.16 101.6) (width 0.25) (layer "F.Cu") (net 10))
 (segment (start 138.43 118.11) (end 133.35 118.11) (width 0.25) (layer "F.Cu") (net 10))
 (segment (start 139.075 115.57) (end 139.075 117.465) (width 0.25) (layer "F.Cu") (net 10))
 (segment (start 133.35 118.11) (end 132.08 116.84) (width 0.25) (layer "F.Cu") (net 10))
 (segment (start 134.62 92.71) (end 137.16 95.25) (width 0.25) (layer "F.Cu") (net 10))
 (segment (start 139.075 117.465) (end 138.43 118.11) (width 0.25) (layer "F.Cu") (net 10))
 (segment (start 132.08 116.84) (end 132.08 114.3) (width 0.25) (layer "F.Cu") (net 10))
 (segment (start 137.16 101.6) (end 137.16 99.06) (width 0.25) (layer "F.Cu") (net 10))
 (segment (start 139.7 106.68) (end 139.7 104.14) (width 0.25) (layer "F.Cu") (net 10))
 (segment (start 133.35 119.38) (end 130.81 116.84) (width 0.25) (layer "F.Cu") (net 9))
 (segment (start 127 91.44) (end 127 92.71) (width 0.25) (layer "F.Cu") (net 9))
 (segment (start 134.62 106.68) (end 134.62 104.14) (width 0.25) (layer "F.Cu") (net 9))
 (segment (start 134.62 104.14) (end 132.08 101.6) (width 0.25) (layer "F.Cu") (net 9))
 (segment (start 132.08 101.6) (end 132.08 99.06) (width 0.25) (layer "F.Cu") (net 9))
 (segment (start 140.325 115.57) (end 140.325 117.485) (width 0.25) (layer "F.Cu") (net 9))
 (segment (start 140.325 117.485) (end 138.43 119.38) (width 0.25) (layer "F.Cu") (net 9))
 (segment (start 132.08 97.79) (end 132.08 99.06) (width 0.25) (layer "F.Cu") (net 9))
 (segment (start 127 92.71) (end 132.08 97.79) (width 0.25) (layer "F.Cu") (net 9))
 (segment (start 138.43 119.38) (end 133.35 119.38) (width 0.25) (layer "F.Cu") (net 9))
 (segment (start 130.81 116.84) (end 130.81 110.49) (width 0.25) (layer "F.Cu") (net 9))
 (segment (start 130.81 110.49) (end 134.62 106.68) (width 0.25) (layer "F.Cu") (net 9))
 (segment (start 124.46 91.44) (end 124.46 92.71) (width 0.25) (layer "F.Cu") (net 8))
 (segment (start 129.54 104.14) (end 129.54 111.76) (width 0.25) (layer "F.Cu") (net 8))
 (segment (start 127 99.06) (end 127 101.6) (width 0.25) (layer "F.Cu") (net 8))
 (segment (start 127 101.6) (end 129.54 104.14) (width 0.25) (layer "F.Cu") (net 8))
 (segment (start 124.46 92.71) (end 127 95.25) (width 0.25) (layer "F.Cu") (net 8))
 (segment (start 127 95.25) (end 127 99.06) (width 0.25) (layer "F.Cu") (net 8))
 (via (at 129.54 111.76) (size 0.8) (drill 0.4) (layers "F.Cu" "B.Cu") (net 8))
 (segment (start 141.575 115.57) (end 141.575 117.505) (width 0.25) (layer "B.Cu") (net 8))
 (segment (start 140.97 118.11) (end 132.08 118.11) (width 0.25) (layer "B.Cu") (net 8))
 (segment (start 132.08 118.11) (end 129.54 115.57) (width 0.25) (layer "B.Cu") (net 8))
 (segment (start 129.54 111.76) (end 129.54 115.57) (width 0.25) (layer "B.Cu") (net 8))
 (segment (start 141.575 117.505) (end 140.97 118.11) (width 0.25) (layer "B.Cu") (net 8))
 (segment (start 116.84 91.44) (end 116.84 92.71) (width 0.25) (layer "F.Cu") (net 6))
 (segment (start 116.84 92.71) (end 121.92 97.79) (width 0.25) (layer "F.Cu") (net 6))
 (segment (start 124.46 110.49) (end 124.46 104.14) (width 0.25) (layer "F.Cu") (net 6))
 (segment (start 121.92 99.06) (end 121.92 101.6) (width 0.25) (layer "F.Cu") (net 6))
 (segment (start 121.92 97.79) (end 121.92 99.06) (width 0.25) (layer "F.Cu") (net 6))
 (segment (start 121.92 101.6) (end 124.46 104.14) (width 0.25) (layer "F.Cu") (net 6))
 (via (at 124.46 110.49) (size 0.8) (drill 0.4) (layers "F.Cu" "B.Cu") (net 6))
 (segment (start 140.97 119.38) (end 130.81 119.38) (width 0.25) (layer "B.Cu") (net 6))
 (segment (start 142.825 117.525) (end 140.97 119.38) (width 0.25) (layer "B.Cu") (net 6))
 (segment (start 142.825 115.57) (end 142.825 117.525) (width 0.25) (layer "B.Cu") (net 6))
 (segment (start 124.46 113.03) (end 124.46 110.49) (width 0.25) (layer "B.Cu") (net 6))
 (segment (start 130.81 119.38) (end 124.46 113.03) (width 0.25) (layer "B.Cu") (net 6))
 (segment (start 147.32 91.44) (end 149.86 91.44) (width 0.25) (layer "B.Cu") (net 7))
 (segment (start 144.78 118.11) (end 144.075 117.405) (width 0.25) (layer "B.Cu") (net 7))
 (segment (start 119.38 91.44) (end 121.92 91.44) (width 0.25) (layer "B.Cu") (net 7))
 (segment (start 157.48 91.44) (end 160.02 91.44) (width 0.25) (layer "B.Cu") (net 7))
 (segment (start 161.29 111.76) (end 154.94 118.11) (width 0.25) (layer "B.Cu") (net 7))
 (segment (start 149.86 91.44) (end 144.78 96.52) (width 0.25) (layer "B.Cu") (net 7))
 (segment (start 144.075 117.405) (end 144.075 115.57) (width 0.25) (layer "B.Cu") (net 7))
 (segment (start 158.75 96.52) (end 161.29 99.06) (width 0.25) (layer "B.Cu") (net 7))
 (segment (start 154.94 96.52) (end 158.75 96.52) (width 0.25) (layer "B.Cu") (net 7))
 (segment (start 154.94 118.11) (end 144.78 118.11) (width 0.25) (layer "B.Cu") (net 7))
 (segment (start 129.54 91.44) (end 134.62 96.52) (width 0.25) (layer "B.Cu") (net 7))
 (segment (start 134.62 96.52) (end 139.7 96.52) (width 0.25) (layer "B.Cu") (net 7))
 (segment (start 139.7 96.52) (end 144.78 96.52) (width 0.25) (layer "B.Cu") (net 7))
 (segment (start 124.46 96.52) (end 134.62 96.52) (width 0.25) (layer "B.Cu") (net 7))
 (segment (start 119.38 91.44) (end 124.46 96.52) (width 0.25) (layer "B.Cu") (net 7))
 (segment (start 129.54 91.44) (end 132.08 91.44) (width 0.25) (layer "B.Cu") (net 7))
 (segment (start 154.94 96.52) (end 160.02 91.44) (width 0.25) (layer "B.Cu") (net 7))
 (segment (start 161.29 99.06) (end 161.29 111.76) (width 0.25) (layer "B.Cu") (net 7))
 (segment (start 144.78 96.52) (end 154.94 96.52) (width 0.25) (layer "B.Cu") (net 7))
 (segment (start 145.325 112.485) (end 145.325 115.57) (width 0.25) (layer "F.Cu") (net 20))
 (segment (start 147.32 110.49) (end 145.325 112.485) (width 0.25) (layer "F.Cu") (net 20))
 (segment (start 147.32 106.68) (end 147.32 110.49) (width 0.25) (layer "F.Cu") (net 20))
 (segment (start 127 106.68) (end 132.08 106.68) (width 0.25) (layer "B.Cu") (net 20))
 (segment (start 147.32 106.68) (end 152.4 106.68) (width 0.25) (layer "B.Cu") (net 20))
 (segment (start 152.4 106.68) (end 157.48 106.68) (width 0.25) (layer "B.Cu") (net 20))
 (segment (start 137.16 106.68) (end 142.24 106.68) (width 0.25) (layer "B.Cu") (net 20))
 (segment (start 121.92 106.68) (end 127 106.68) (width 0.25) (layer "B.Cu") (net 20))
 (segment (start 142.24 106.68) (end 147.32 106.68) (width 0.25) (layer "B.Cu") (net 20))
 (segment (start 132.08 106.68) (end 137.16 106.68) (width 0.25) (layer "B.Cu") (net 20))
 (segment (start 162.56 82.55) (end 162.56 83.82) (width 0.25) (layer "F.Cu") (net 22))
 (segment (start 157.48 76.2) (end 157.48 77.47) (width 0.25) (layer "F.Cu") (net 22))
 (segment (start 157.48 77.47) (end 162.56 82.55) (width 0.25) (layer "F.Cu") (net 22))
 (segment (start 152.4 77.47) (end 154.94 80.01) (width 0.25) (layer "F.Cu") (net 23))
 (segment (start 154.94 80.01) (end 154.94 83.82) (width 0.25) (layer "F.Cu") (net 23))
 (segment (start 152.4 76.2) (end 152.4 77.47) (width 0.25) (layer "F.Cu") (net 23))
 (segment (start 147.32 77.47) (end 152.4 82.55) (width 0.25) (layer "F.Cu") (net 24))
 (segment (start 147.32 76.2) (end 147.32 77.47) (width 0.25) (layer "F.Cu") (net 24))
 (segment (start 152.4 82.55) (end 152.4 83.82) (width 0.25) (layer "F.Cu") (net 24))
 (segment (start 144.78 80.01) (end 144.78 83.82) (width 0.25) (layer "F.Cu") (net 13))
 (segment (start 142.24 76.2) (end 142.24 77.47) (width 0.25) (layer "F.Cu") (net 13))
 (segment (start 142.24 77.47) (end 144.78 80.01) (width 0.25) (layer "F.Cu") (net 13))
 (segment (start 134.62 80.01) (end 134.62 83.82) (width 0.25) (layer "F.Cu") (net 1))
 (segment (start 137.16 77.47) (end 134.62 80.01) (width 0.25) (layer "F.Cu") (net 1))
 (segment (start 137.16 76.2) (end 137.16 77.47) (width 0.25) (layer "F.Cu") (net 1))
 (segment (start 127 82.55) (end 127 83.82) (width 0.25) (layer "F.Cu") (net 3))
 (segment (start 132.08 77.47) (end 127 82.55) (width 0.25) (layer "F.Cu") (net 3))
 (segment (start 132.08 76.2) (end 132.08 77.47) (width 0.25) (layer "F.Cu") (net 3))
 (segment (start 127 77.47) (end 124.46 80.01) (width 0.25) (layer "F.Cu") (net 4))
 (segment (start 127 76.2) (end 127 77.47) (width 0.25) (layer "F.Cu") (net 4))
 (segment (start 124.46 80.01) (end 124.46 83.82) (width 0.25) (layer "F.Cu") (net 4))
 (segment (start 121.92 76.2) (end 121.92 77.47) (width 0.25) (layer "F.Cu") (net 5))
 (segment (start 116.84 82.55) (end 116.84 83.82) (width 0.25) (layer "F.Cu") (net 5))
 (segment (start 121.92 77.47) (end 116.84 82.55) (width 0.25) (layer "F.Cu") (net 5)))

